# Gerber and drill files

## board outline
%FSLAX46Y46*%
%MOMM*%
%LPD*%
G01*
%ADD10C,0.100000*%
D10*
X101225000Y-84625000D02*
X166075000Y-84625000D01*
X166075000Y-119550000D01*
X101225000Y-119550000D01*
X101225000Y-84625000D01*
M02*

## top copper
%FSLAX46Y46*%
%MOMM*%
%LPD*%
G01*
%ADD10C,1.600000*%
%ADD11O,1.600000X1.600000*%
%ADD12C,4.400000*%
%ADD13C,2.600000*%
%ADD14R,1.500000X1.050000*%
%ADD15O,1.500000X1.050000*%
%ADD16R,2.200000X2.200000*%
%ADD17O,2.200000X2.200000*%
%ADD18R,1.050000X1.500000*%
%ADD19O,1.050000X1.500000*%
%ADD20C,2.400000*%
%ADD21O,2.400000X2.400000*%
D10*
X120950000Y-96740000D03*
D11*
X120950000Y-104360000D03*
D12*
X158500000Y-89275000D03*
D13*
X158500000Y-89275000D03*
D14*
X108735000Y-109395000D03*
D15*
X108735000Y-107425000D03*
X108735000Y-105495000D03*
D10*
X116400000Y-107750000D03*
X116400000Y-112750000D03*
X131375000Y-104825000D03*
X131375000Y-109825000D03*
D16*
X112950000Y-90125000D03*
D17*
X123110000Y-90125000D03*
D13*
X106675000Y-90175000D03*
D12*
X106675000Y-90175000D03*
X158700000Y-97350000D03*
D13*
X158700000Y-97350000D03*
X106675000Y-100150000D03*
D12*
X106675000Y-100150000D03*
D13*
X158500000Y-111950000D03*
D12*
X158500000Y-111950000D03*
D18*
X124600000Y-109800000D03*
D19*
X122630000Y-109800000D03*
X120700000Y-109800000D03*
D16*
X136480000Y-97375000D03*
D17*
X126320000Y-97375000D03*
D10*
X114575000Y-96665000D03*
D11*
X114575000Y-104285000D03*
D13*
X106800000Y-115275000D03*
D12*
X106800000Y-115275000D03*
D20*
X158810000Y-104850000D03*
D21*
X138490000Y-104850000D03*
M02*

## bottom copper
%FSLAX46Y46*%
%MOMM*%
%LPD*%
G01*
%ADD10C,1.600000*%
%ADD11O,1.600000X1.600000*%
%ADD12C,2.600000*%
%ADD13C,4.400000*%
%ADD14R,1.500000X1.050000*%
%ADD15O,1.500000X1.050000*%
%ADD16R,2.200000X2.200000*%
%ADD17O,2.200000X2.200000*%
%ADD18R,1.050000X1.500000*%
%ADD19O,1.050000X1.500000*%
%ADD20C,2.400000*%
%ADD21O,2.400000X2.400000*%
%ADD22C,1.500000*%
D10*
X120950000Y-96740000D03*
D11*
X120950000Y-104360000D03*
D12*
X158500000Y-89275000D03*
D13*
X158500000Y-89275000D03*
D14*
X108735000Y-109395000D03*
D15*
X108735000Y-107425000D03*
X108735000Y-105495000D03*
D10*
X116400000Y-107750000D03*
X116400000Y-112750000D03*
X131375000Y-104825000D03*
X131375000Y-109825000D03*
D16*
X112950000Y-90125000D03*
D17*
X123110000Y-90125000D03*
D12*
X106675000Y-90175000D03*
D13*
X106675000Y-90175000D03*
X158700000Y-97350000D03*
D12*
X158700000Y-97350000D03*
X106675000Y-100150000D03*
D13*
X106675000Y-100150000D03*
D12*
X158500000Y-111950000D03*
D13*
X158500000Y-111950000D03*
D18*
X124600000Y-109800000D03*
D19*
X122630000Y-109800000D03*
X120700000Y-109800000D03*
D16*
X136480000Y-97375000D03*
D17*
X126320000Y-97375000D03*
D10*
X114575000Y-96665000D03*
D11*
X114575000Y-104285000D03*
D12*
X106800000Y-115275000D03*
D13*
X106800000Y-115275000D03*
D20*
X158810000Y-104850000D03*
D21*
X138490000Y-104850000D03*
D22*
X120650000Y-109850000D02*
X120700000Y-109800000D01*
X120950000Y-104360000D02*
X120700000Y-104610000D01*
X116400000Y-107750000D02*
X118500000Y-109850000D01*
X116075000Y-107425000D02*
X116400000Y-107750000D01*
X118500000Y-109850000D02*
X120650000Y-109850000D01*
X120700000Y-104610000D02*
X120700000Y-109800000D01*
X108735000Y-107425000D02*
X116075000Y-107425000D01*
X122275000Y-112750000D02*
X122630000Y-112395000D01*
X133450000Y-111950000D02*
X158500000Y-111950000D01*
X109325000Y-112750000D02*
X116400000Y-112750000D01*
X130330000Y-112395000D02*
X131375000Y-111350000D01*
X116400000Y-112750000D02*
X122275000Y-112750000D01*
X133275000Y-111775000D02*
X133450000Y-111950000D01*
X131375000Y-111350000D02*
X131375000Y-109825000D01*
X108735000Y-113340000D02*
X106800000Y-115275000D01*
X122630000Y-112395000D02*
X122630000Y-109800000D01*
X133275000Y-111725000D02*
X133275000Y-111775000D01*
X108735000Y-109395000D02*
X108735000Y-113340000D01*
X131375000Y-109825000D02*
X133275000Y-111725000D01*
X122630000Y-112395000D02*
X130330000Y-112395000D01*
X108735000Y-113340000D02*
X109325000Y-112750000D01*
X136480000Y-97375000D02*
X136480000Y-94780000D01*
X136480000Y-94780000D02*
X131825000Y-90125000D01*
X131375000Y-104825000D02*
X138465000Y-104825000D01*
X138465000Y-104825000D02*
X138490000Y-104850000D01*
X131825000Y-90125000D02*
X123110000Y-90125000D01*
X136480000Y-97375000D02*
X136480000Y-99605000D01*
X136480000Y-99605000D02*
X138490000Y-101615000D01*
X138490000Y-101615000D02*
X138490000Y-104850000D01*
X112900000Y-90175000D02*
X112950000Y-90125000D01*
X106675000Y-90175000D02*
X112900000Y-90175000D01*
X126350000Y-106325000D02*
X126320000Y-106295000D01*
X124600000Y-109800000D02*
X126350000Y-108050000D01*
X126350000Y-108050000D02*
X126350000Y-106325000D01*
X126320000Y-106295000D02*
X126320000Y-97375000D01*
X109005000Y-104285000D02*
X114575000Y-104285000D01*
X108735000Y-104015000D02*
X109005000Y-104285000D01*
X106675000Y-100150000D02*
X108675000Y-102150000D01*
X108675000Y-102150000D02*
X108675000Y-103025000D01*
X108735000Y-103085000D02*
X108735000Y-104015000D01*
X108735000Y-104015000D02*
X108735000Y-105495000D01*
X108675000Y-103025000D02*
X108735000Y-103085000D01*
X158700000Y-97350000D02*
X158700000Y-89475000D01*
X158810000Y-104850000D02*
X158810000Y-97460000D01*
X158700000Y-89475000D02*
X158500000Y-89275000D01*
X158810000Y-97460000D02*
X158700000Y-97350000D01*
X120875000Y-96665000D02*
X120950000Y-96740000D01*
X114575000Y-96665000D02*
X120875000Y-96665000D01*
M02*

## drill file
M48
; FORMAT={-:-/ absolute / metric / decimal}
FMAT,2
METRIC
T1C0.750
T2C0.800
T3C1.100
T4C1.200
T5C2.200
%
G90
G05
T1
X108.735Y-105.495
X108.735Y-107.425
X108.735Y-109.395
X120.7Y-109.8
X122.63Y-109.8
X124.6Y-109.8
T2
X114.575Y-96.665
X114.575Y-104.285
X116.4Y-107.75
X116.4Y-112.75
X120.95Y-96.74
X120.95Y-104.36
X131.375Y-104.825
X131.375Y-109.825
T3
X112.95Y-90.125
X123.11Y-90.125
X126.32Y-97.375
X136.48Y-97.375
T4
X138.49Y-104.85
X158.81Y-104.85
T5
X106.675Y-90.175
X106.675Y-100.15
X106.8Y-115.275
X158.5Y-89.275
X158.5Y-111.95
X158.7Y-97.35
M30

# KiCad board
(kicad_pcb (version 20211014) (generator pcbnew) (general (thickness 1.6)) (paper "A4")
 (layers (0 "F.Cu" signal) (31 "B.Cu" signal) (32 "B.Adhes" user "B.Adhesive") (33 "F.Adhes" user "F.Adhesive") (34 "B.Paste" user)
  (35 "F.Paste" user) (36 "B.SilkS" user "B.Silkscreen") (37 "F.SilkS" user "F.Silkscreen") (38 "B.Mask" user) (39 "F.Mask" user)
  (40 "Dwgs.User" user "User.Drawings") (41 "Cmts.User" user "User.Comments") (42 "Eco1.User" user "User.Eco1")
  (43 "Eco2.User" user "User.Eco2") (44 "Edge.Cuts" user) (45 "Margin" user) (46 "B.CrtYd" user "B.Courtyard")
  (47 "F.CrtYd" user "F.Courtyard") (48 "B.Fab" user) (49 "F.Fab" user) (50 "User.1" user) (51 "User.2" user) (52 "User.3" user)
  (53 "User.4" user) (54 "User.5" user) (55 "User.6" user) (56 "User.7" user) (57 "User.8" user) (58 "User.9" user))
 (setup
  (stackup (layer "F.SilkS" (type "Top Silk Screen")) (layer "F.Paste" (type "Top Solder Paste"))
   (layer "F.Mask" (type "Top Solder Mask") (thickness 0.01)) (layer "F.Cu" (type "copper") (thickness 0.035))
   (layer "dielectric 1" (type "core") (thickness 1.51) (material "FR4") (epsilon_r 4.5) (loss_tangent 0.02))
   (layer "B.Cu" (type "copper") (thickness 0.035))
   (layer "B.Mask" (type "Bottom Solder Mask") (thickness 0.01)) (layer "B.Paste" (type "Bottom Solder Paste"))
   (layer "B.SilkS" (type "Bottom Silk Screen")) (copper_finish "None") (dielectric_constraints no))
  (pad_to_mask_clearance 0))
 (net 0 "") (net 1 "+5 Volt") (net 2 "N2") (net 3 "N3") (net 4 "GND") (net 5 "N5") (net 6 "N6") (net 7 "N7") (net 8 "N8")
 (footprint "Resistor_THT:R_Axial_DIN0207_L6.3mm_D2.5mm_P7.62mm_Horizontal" (layer "F.Cu") (at 120.95 96.74 -90)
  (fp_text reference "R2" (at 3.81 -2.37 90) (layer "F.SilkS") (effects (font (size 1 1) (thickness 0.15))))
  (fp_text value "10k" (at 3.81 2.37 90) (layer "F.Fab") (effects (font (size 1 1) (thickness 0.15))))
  (pad "1" thru_hole circle (at 0 0 270) (size 1.6 1.6) (drill 0.8) (layers *.Cu *.Mask) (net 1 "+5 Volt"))
  (pad "2" thru_hole oval (at 7.62 0 270) (size 1.6 1.6) (drill 0.8) (layers *.Cu *.Mask) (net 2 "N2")))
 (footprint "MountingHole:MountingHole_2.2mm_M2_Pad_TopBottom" (layer "F.Cu") (at 158.5 89.275)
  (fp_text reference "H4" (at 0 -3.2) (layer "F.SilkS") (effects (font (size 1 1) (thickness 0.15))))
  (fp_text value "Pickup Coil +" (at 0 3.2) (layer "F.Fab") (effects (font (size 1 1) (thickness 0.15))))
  (pad "1" connect circle (at 0 0) (size 4.4 4.4) (layers "F.Cu" "F.Mask") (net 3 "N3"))
  (pad "1" thru_hole circle (at 0 0) (size 2.6 2.6) (drill 2.2) (layers *.Cu *.Mask) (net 3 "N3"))
  (pad "1" connect circle (at 0 0) (size 4.4 4.4) (layers "B.Cu" "B.Mask") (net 3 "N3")))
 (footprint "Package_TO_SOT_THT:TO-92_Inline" (layer "F.Cu") (at 108.735 108.695 90)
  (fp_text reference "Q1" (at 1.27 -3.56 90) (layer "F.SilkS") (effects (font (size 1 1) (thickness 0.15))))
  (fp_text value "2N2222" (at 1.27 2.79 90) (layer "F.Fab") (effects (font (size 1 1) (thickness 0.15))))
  (pad "1" thru_hole rect (at -0.7 0 90) (size 1.05 1.5) (drill 0.75) (layers *.Cu *.Mask) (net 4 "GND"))
  (pad "2" thru_hole oval (at 1.27 0 90) (size 1.05 1.5) (drill 0.75) (layers *.Cu *.Mask) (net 2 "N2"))
  (pad "3" thru_hole oval (at 3.2 0 90) (size 1.05 1.5) (drill 0.75) (layers *.Cu *.Mask) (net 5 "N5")))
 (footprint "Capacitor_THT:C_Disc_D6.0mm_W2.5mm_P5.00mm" (layer "F.Cu") (at 116.4 107.75 -90)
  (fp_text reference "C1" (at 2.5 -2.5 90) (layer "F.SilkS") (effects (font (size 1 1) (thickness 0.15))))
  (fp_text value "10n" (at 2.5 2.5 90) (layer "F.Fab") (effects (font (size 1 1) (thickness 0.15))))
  (pad "1" thru_hole circle (at 0 0 270) (size 1.6 1.6) (drill 0.8) (layers *.Cu *.Mask) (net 2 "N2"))
  (pad "2" thru_hole circle (at 5 0 270) (size 1.6 1.6) (drill 0.8) (layers *.Cu *.Mask) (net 4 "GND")))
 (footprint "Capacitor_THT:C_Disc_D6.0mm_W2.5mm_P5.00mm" (layer "F.Cu") (at 131.375 104.825 -90)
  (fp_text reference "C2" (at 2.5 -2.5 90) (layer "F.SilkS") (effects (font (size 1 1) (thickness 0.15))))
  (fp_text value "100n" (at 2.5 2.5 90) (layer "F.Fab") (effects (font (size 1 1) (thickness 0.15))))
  (pad "1" thru_hole circle (at 0 0 270) (size 1.6 1.6) (drill 0.8) (layers *.Cu *.Mask) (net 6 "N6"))
  (pad "2" thru_hole circle (at 5 0 270) (size 1.6 1.6) (drill 0.8) (layers *.Cu *.Mask) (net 4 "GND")))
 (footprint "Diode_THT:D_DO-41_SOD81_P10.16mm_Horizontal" (layer "F.Cu") (at 112.95 90.125)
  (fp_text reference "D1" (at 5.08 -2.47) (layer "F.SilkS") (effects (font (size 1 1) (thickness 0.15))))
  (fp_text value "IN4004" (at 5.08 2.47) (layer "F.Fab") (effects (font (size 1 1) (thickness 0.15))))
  (pad "1" thru_hole rect (at 0 0) (size 2.2 2.2) (drill 1.1) (layers *.Cu *.Mask) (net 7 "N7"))
  (pad "2" thru_hole oval (at 10.16 0) (size 2.2 2.2) (drill 1.1) (layers *.Cu *.Mask) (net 6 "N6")))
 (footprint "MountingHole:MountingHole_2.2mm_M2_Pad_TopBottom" (layer "F.Cu") (at 106.675 90.175)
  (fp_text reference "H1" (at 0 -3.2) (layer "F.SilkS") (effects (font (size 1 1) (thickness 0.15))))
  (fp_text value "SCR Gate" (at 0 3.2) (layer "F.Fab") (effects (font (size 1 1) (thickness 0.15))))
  (pad "1" thru_hole circle (at 0 0) (size 2.6 2.6) (drill 2.2) (layers *.Cu *.Mask) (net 7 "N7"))
  (pad "1" connect circle (at 0 0) (size 4.4 4.4) (layers "B.Cu" "B.Mask") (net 7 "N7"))
  (pad "1" connect circle (at 0 0) (size 4.4 4.4) (layers "F.Cu" "F.Mask") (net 7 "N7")))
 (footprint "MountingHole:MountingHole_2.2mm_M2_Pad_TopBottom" (layer "F.Cu") (at 158.7 97.35)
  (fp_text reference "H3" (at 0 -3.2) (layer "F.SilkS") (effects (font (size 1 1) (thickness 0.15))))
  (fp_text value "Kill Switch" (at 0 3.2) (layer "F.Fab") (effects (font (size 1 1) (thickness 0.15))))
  (pad "1" connect circle (at 0 0) (size 4.4 4.4) (layers "B.Cu" "B.Mask") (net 3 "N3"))
  (pad "1" connect circle (at 0 0) (size 4.4 4.4) (layers "F.Cu" "F.Mask") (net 3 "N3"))
  (pad "1" thru_hole circle (at 0 0) (size 2.6 2.6) (drill 2.2) (layers *.Cu *.Mask) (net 3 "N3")))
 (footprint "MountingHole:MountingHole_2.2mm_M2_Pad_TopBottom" (layer "F.Cu") (at 106.675 100.15)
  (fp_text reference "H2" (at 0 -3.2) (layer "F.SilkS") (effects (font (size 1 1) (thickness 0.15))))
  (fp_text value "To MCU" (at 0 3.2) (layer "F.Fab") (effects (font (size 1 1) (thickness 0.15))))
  (pad "1" thru_hole circle (at 0 0) (size 2.6 2.6) (drill 2.2) (layers *.Cu *.Mask) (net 5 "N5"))
  (pad "1" connect circle (at 0 0) (size 4.4 4.4) (layers "F.Cu" "F.Mask") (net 5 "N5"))
  (pad "1" connect circle (at 0 0) (size 4.4 4.4) (layers "B.Cu" "B.Mask") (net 5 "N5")))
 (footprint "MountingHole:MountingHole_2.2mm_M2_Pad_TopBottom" (layer "F.Cu") (at 158.5 111.95)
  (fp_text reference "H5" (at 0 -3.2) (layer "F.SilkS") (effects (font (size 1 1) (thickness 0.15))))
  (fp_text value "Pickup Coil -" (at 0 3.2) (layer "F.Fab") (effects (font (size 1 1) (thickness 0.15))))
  (pad "1" thru_hole circle (at 0 0) (size 2.6 2.6) (drill 2.2) (layers *.Cu *.Mask) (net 4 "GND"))
  (pad "1" connect circle (at 0 0) (size 4.4 4.4) (layers "B.Cu" "B.Mask") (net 4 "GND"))
  (pad "1" connect circle (at 0 0) (size 4.4 4.4) (layers "F.Cu" "F.Mask") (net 4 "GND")))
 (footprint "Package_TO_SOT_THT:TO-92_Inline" (layer "F.Cu") (at 123.9 109.8 180)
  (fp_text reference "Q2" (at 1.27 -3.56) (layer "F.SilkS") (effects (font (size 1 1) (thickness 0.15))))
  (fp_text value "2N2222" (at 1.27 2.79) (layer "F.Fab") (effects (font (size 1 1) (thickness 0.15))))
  (pad "1" thru_hole rect (at -0.7 0 180) (size 1.05 1.5) (drill 0.75) (layers *.Cu *.Mask) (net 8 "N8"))
  (pad "2" thru_hole oval (at 1.27 0 180) (size 1.05 1.5) (drill 0.75) (layers *.Cu *.Mask) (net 4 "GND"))
  (pad "3" thru_hole oval (at 3.2 0 180) (size 1.05 1.5) (drill 0.75) (layers *.Cu *.Mask) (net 2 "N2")))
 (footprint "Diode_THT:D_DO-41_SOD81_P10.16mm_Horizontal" (layer "F.Cu") (at 136.48 97.375 180)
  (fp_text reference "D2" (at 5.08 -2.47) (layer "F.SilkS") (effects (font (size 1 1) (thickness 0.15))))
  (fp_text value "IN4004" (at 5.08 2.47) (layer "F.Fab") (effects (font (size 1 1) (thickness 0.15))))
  (pad "1" thru_hole rect (at 0 0 180) (size 2.2 2.2) (drill 1.1) (layers *.Cu *.Mask) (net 6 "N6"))
  (pad "2" thru_hole oval (at 10.16 0 180) (size 2.2 2.2) (drill 1.1) (layers *.Cu *.Mask) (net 8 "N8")))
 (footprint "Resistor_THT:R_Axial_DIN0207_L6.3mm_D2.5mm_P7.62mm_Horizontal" (layer "F.Cu") (at 114.575 96.665 -90)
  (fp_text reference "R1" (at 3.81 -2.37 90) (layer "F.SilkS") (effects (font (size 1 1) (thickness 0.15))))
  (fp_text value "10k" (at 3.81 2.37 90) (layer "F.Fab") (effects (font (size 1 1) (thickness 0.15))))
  (pad "1" thru_hole circle (at 0 0 270) (size 1.6 1.6) (drill 0.8) (layers *.Cu *.Mask) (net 1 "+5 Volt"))
  (pad "2" thru_hole oval (at 7.62 0 270) (size 1.6 1.6) (drill 0.8) (layers *.Cu *.Mask) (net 5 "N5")))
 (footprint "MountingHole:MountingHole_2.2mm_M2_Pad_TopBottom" (layer "F.Cu") (at 106.8 115.275)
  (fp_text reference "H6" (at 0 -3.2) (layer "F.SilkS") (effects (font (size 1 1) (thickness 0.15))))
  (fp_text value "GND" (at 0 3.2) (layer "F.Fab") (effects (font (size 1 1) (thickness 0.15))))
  (pad "1" thru_hole circle (at 0 0) (size 2.6 2.6) (drill 2.2) (layers *.Cu *.Mask) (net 4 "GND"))
  (pad "1" connect circle (at 0 0) (size 4.4 4.4) (layers "B.Cu" "B.Mask") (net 4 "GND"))
  (pad "1" connect circle (at 0 0) (size 4.4 4.4) (layers "F.Cu" "F.Mask") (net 4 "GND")))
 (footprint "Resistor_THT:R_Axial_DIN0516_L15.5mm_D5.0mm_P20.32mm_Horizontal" (layer "F.Cu") (at 158.81 104.85 180)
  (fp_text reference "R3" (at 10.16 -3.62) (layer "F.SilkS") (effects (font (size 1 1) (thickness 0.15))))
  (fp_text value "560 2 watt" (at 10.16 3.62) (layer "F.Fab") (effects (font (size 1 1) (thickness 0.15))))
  (pad "1" thru_hole circle (at 0 0 180) (size 2.4 2.4) (drill 1.2) (layers *.Cu *.Mask) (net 3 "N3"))
  (pad "2" thru_hole oval (at 20.32 0 180) (size 2.4 2.4) (drill 1.2) (layers *.Cu *.Mask) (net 6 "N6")))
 (gr_rect (start 101.225 84.625) (end 166.075 119.55) (layer "Edge.Cuts") (width 0.1) (fill none))
 (segment (start 120.65 109.85) (end 120.7 109.8) (width 1.5) (layer "B.Cu") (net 2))
 (segment (start 120.95 104.36) (end 120.7 104.61) (width 1.5) (layer "B.Cu") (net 2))
 (segment (start 116.4 107.75) (end 118.5 109.85) (width 1.5) (layer "B.Cu") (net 2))
 (segment (start 116.075 107.425) (end 116.4 107.75) (width 1.5) (layer "B.Cu") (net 2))
 (segment (start 118.5 109.85) (end 120.65 109.85) (width 1.5) (layer "B.Cu") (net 2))
 (segment (start 120.7 104.61) (end 120.7 109.8) (width 1.5) (layer "B.Cu") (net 2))
 (segment (start 108.735 107.425) (end 116.075 107.425) (width 1.5) (layer "B.Cu") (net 2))
 (segment (start 122.275 112.75) (end 122.63 112.395) (width 1.5) (layer "B.Cu") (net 4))
 (segment (start 133.45 111.95) (end 158.5 111.95) (width 1.5) (layer "B.Cu") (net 4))
 (segment (start 109.325 112.75) (end 116.4 112.75) (width 1.5) (layer "B.Cu") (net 4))
 (segment (start 130.33 112.395) (end 131.375 111.35) (width 1.5) (layer "B.Cu") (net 4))
 (segment (start 116.4 112.75) (end 122.275 112.75) (width 1.5) (layer "B.Cu") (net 4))
 (segment (start 133.275 111.775) (end 133.45 111.95) (width 1.5) (layer "B.Cu") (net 4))
 (segment (start 131.375 111.35) (end 131.375 109.825) (width 1.5) (layer "B.Cu") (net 4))
 (segment (start 108.735 113.34) (end 106.8 115.275) (width 1.5) (layer "B.Cu") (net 4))
 (segment (start 122.63 112.395) (end 122.63 109.8) (width 1.5) (layer "B.Cu") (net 4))
 (segment (start 133.275 111.725) (end 133.275 111.775) (width 1.5) (layer "B.Cu") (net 4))
 (segment (start 108.735 109.395) (end 108.735 113.34) (width 1.5) (layer "B.Cu") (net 4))
 (segment (start 131.375 109.825) (end 133.275 111.725) (width 1.5) (layer "B.Cu") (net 4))
 (segment (start 122.63 112.395) (end 130.33 112.395) (width 1.5) (layer "B.Cu") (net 4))
 (segment (start 108.735 113.34) (end 109.325 112.75) (width 1.5) (layer "B.Cu") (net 4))
 (segment (start 136.48 97.375) (end 136.48 94.78) (width 1.5) (layer "B.Cu") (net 6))
 (segment (start 136.48 94.78) (end 131.825 90.125) (width 1.5) (layer "B.Cu") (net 6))
 (segment (start 131.375 104.825) (end 138.465 104.825) (width 1.5) (layer "B.Cu") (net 6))
 (segment (start 138.465 104.825) (end 138.49 104.85) (width 1.5) (layer "B.Cu") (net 6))
 (segment (start 131.825 90.125) (end 123.11 90.125) (width 1.5) (layer "B.Cu") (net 6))
 (segment (start 136.48 97.375) (end 136.48 99.605) (width 1.5) (layer "B.Cu") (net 6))
 (segment (start 136.48 99.605) (end 138.49 101.615) (width 1.5) (layer "B.Cu") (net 6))
 (segment (start 138.49 101.615) (end 138.49 104.85) (width 1.5) (layer "B.Cu") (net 6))
 (segment (start 112.9 90.175) (end 112.95 90.125) (width 1.5) (layer "B.Cu") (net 7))
 (segment (start 106.675 90.175) (end 112.9 90.175) (width 1.5) (layer "B.Cu") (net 7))
 (segment (start 126.35 106.325) (end 126.32 106.295) (width 1.5) (layer "B.Cu") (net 8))
 (segment (start 124.6 109.8) (end 126.35 108.05) (width 1.5) (layer "B.Cu") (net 8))
 (segment (start 126.35 108.05) (end 126.35 106.325) (width 1.5) (layer "B.Cu") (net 8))
 (segment (start 126.32 106.295) (end 126.32 97.375) (width 1.5) (layer "B.Cu") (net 8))
 (segment (start 109.005 104.285) (end 114.575 104.285) (width 1.5) (layer "B.Cu") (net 5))
 (segment (start 108.735 104.015) (end 109.005 104.285) (width 1.5) (layer "B.Cu") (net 5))
 (segment (start 106.675 100.15) (end 108.675 102.15) (width 1.5) (layer "B.Cu") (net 5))
 (segment (start 108.675 102.15) (end 108.675 103.025) (width 1.5) (layer "B.Cu") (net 5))
 (segment (start 108.735 103.085) (end 108.735 104.015) (width 1.5) (layer "B.Cu") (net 5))
 (segment (start 108.735 104.015) (end 108.735 105.495) (width 1.5) (layer "B.Cu") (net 5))
 (segment (start 108.675 103.025) (end 108.735 103.085) (width 1.5) (layer "B.Cu") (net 5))
 (segment (start 158.7 97.35) (end 158.7 89.475) (width 1.5) (layer "B.Cu") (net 3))
 (segment (start 158.81 104.85) (end 158.81 97.46) (width 1.5) (layer "B.Cu") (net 3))
 (segment (start 158.7 89.475) (end 158.5 89.275) (width 1.5) (layer "B.Cu") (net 3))
 (segment (start 158.81 97.46) (end 158.7 97.35) (width 1.5) (layer "B.Cu") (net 3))
 (segment (start 120.875 96.665) (end 120.95 96.74) (width 1.5) (layer "B.Cu") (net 1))
 (segment (start 114.575 96.665) (end 120.875 96.665) (width 1.5) (layer "B.Cu") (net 1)))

